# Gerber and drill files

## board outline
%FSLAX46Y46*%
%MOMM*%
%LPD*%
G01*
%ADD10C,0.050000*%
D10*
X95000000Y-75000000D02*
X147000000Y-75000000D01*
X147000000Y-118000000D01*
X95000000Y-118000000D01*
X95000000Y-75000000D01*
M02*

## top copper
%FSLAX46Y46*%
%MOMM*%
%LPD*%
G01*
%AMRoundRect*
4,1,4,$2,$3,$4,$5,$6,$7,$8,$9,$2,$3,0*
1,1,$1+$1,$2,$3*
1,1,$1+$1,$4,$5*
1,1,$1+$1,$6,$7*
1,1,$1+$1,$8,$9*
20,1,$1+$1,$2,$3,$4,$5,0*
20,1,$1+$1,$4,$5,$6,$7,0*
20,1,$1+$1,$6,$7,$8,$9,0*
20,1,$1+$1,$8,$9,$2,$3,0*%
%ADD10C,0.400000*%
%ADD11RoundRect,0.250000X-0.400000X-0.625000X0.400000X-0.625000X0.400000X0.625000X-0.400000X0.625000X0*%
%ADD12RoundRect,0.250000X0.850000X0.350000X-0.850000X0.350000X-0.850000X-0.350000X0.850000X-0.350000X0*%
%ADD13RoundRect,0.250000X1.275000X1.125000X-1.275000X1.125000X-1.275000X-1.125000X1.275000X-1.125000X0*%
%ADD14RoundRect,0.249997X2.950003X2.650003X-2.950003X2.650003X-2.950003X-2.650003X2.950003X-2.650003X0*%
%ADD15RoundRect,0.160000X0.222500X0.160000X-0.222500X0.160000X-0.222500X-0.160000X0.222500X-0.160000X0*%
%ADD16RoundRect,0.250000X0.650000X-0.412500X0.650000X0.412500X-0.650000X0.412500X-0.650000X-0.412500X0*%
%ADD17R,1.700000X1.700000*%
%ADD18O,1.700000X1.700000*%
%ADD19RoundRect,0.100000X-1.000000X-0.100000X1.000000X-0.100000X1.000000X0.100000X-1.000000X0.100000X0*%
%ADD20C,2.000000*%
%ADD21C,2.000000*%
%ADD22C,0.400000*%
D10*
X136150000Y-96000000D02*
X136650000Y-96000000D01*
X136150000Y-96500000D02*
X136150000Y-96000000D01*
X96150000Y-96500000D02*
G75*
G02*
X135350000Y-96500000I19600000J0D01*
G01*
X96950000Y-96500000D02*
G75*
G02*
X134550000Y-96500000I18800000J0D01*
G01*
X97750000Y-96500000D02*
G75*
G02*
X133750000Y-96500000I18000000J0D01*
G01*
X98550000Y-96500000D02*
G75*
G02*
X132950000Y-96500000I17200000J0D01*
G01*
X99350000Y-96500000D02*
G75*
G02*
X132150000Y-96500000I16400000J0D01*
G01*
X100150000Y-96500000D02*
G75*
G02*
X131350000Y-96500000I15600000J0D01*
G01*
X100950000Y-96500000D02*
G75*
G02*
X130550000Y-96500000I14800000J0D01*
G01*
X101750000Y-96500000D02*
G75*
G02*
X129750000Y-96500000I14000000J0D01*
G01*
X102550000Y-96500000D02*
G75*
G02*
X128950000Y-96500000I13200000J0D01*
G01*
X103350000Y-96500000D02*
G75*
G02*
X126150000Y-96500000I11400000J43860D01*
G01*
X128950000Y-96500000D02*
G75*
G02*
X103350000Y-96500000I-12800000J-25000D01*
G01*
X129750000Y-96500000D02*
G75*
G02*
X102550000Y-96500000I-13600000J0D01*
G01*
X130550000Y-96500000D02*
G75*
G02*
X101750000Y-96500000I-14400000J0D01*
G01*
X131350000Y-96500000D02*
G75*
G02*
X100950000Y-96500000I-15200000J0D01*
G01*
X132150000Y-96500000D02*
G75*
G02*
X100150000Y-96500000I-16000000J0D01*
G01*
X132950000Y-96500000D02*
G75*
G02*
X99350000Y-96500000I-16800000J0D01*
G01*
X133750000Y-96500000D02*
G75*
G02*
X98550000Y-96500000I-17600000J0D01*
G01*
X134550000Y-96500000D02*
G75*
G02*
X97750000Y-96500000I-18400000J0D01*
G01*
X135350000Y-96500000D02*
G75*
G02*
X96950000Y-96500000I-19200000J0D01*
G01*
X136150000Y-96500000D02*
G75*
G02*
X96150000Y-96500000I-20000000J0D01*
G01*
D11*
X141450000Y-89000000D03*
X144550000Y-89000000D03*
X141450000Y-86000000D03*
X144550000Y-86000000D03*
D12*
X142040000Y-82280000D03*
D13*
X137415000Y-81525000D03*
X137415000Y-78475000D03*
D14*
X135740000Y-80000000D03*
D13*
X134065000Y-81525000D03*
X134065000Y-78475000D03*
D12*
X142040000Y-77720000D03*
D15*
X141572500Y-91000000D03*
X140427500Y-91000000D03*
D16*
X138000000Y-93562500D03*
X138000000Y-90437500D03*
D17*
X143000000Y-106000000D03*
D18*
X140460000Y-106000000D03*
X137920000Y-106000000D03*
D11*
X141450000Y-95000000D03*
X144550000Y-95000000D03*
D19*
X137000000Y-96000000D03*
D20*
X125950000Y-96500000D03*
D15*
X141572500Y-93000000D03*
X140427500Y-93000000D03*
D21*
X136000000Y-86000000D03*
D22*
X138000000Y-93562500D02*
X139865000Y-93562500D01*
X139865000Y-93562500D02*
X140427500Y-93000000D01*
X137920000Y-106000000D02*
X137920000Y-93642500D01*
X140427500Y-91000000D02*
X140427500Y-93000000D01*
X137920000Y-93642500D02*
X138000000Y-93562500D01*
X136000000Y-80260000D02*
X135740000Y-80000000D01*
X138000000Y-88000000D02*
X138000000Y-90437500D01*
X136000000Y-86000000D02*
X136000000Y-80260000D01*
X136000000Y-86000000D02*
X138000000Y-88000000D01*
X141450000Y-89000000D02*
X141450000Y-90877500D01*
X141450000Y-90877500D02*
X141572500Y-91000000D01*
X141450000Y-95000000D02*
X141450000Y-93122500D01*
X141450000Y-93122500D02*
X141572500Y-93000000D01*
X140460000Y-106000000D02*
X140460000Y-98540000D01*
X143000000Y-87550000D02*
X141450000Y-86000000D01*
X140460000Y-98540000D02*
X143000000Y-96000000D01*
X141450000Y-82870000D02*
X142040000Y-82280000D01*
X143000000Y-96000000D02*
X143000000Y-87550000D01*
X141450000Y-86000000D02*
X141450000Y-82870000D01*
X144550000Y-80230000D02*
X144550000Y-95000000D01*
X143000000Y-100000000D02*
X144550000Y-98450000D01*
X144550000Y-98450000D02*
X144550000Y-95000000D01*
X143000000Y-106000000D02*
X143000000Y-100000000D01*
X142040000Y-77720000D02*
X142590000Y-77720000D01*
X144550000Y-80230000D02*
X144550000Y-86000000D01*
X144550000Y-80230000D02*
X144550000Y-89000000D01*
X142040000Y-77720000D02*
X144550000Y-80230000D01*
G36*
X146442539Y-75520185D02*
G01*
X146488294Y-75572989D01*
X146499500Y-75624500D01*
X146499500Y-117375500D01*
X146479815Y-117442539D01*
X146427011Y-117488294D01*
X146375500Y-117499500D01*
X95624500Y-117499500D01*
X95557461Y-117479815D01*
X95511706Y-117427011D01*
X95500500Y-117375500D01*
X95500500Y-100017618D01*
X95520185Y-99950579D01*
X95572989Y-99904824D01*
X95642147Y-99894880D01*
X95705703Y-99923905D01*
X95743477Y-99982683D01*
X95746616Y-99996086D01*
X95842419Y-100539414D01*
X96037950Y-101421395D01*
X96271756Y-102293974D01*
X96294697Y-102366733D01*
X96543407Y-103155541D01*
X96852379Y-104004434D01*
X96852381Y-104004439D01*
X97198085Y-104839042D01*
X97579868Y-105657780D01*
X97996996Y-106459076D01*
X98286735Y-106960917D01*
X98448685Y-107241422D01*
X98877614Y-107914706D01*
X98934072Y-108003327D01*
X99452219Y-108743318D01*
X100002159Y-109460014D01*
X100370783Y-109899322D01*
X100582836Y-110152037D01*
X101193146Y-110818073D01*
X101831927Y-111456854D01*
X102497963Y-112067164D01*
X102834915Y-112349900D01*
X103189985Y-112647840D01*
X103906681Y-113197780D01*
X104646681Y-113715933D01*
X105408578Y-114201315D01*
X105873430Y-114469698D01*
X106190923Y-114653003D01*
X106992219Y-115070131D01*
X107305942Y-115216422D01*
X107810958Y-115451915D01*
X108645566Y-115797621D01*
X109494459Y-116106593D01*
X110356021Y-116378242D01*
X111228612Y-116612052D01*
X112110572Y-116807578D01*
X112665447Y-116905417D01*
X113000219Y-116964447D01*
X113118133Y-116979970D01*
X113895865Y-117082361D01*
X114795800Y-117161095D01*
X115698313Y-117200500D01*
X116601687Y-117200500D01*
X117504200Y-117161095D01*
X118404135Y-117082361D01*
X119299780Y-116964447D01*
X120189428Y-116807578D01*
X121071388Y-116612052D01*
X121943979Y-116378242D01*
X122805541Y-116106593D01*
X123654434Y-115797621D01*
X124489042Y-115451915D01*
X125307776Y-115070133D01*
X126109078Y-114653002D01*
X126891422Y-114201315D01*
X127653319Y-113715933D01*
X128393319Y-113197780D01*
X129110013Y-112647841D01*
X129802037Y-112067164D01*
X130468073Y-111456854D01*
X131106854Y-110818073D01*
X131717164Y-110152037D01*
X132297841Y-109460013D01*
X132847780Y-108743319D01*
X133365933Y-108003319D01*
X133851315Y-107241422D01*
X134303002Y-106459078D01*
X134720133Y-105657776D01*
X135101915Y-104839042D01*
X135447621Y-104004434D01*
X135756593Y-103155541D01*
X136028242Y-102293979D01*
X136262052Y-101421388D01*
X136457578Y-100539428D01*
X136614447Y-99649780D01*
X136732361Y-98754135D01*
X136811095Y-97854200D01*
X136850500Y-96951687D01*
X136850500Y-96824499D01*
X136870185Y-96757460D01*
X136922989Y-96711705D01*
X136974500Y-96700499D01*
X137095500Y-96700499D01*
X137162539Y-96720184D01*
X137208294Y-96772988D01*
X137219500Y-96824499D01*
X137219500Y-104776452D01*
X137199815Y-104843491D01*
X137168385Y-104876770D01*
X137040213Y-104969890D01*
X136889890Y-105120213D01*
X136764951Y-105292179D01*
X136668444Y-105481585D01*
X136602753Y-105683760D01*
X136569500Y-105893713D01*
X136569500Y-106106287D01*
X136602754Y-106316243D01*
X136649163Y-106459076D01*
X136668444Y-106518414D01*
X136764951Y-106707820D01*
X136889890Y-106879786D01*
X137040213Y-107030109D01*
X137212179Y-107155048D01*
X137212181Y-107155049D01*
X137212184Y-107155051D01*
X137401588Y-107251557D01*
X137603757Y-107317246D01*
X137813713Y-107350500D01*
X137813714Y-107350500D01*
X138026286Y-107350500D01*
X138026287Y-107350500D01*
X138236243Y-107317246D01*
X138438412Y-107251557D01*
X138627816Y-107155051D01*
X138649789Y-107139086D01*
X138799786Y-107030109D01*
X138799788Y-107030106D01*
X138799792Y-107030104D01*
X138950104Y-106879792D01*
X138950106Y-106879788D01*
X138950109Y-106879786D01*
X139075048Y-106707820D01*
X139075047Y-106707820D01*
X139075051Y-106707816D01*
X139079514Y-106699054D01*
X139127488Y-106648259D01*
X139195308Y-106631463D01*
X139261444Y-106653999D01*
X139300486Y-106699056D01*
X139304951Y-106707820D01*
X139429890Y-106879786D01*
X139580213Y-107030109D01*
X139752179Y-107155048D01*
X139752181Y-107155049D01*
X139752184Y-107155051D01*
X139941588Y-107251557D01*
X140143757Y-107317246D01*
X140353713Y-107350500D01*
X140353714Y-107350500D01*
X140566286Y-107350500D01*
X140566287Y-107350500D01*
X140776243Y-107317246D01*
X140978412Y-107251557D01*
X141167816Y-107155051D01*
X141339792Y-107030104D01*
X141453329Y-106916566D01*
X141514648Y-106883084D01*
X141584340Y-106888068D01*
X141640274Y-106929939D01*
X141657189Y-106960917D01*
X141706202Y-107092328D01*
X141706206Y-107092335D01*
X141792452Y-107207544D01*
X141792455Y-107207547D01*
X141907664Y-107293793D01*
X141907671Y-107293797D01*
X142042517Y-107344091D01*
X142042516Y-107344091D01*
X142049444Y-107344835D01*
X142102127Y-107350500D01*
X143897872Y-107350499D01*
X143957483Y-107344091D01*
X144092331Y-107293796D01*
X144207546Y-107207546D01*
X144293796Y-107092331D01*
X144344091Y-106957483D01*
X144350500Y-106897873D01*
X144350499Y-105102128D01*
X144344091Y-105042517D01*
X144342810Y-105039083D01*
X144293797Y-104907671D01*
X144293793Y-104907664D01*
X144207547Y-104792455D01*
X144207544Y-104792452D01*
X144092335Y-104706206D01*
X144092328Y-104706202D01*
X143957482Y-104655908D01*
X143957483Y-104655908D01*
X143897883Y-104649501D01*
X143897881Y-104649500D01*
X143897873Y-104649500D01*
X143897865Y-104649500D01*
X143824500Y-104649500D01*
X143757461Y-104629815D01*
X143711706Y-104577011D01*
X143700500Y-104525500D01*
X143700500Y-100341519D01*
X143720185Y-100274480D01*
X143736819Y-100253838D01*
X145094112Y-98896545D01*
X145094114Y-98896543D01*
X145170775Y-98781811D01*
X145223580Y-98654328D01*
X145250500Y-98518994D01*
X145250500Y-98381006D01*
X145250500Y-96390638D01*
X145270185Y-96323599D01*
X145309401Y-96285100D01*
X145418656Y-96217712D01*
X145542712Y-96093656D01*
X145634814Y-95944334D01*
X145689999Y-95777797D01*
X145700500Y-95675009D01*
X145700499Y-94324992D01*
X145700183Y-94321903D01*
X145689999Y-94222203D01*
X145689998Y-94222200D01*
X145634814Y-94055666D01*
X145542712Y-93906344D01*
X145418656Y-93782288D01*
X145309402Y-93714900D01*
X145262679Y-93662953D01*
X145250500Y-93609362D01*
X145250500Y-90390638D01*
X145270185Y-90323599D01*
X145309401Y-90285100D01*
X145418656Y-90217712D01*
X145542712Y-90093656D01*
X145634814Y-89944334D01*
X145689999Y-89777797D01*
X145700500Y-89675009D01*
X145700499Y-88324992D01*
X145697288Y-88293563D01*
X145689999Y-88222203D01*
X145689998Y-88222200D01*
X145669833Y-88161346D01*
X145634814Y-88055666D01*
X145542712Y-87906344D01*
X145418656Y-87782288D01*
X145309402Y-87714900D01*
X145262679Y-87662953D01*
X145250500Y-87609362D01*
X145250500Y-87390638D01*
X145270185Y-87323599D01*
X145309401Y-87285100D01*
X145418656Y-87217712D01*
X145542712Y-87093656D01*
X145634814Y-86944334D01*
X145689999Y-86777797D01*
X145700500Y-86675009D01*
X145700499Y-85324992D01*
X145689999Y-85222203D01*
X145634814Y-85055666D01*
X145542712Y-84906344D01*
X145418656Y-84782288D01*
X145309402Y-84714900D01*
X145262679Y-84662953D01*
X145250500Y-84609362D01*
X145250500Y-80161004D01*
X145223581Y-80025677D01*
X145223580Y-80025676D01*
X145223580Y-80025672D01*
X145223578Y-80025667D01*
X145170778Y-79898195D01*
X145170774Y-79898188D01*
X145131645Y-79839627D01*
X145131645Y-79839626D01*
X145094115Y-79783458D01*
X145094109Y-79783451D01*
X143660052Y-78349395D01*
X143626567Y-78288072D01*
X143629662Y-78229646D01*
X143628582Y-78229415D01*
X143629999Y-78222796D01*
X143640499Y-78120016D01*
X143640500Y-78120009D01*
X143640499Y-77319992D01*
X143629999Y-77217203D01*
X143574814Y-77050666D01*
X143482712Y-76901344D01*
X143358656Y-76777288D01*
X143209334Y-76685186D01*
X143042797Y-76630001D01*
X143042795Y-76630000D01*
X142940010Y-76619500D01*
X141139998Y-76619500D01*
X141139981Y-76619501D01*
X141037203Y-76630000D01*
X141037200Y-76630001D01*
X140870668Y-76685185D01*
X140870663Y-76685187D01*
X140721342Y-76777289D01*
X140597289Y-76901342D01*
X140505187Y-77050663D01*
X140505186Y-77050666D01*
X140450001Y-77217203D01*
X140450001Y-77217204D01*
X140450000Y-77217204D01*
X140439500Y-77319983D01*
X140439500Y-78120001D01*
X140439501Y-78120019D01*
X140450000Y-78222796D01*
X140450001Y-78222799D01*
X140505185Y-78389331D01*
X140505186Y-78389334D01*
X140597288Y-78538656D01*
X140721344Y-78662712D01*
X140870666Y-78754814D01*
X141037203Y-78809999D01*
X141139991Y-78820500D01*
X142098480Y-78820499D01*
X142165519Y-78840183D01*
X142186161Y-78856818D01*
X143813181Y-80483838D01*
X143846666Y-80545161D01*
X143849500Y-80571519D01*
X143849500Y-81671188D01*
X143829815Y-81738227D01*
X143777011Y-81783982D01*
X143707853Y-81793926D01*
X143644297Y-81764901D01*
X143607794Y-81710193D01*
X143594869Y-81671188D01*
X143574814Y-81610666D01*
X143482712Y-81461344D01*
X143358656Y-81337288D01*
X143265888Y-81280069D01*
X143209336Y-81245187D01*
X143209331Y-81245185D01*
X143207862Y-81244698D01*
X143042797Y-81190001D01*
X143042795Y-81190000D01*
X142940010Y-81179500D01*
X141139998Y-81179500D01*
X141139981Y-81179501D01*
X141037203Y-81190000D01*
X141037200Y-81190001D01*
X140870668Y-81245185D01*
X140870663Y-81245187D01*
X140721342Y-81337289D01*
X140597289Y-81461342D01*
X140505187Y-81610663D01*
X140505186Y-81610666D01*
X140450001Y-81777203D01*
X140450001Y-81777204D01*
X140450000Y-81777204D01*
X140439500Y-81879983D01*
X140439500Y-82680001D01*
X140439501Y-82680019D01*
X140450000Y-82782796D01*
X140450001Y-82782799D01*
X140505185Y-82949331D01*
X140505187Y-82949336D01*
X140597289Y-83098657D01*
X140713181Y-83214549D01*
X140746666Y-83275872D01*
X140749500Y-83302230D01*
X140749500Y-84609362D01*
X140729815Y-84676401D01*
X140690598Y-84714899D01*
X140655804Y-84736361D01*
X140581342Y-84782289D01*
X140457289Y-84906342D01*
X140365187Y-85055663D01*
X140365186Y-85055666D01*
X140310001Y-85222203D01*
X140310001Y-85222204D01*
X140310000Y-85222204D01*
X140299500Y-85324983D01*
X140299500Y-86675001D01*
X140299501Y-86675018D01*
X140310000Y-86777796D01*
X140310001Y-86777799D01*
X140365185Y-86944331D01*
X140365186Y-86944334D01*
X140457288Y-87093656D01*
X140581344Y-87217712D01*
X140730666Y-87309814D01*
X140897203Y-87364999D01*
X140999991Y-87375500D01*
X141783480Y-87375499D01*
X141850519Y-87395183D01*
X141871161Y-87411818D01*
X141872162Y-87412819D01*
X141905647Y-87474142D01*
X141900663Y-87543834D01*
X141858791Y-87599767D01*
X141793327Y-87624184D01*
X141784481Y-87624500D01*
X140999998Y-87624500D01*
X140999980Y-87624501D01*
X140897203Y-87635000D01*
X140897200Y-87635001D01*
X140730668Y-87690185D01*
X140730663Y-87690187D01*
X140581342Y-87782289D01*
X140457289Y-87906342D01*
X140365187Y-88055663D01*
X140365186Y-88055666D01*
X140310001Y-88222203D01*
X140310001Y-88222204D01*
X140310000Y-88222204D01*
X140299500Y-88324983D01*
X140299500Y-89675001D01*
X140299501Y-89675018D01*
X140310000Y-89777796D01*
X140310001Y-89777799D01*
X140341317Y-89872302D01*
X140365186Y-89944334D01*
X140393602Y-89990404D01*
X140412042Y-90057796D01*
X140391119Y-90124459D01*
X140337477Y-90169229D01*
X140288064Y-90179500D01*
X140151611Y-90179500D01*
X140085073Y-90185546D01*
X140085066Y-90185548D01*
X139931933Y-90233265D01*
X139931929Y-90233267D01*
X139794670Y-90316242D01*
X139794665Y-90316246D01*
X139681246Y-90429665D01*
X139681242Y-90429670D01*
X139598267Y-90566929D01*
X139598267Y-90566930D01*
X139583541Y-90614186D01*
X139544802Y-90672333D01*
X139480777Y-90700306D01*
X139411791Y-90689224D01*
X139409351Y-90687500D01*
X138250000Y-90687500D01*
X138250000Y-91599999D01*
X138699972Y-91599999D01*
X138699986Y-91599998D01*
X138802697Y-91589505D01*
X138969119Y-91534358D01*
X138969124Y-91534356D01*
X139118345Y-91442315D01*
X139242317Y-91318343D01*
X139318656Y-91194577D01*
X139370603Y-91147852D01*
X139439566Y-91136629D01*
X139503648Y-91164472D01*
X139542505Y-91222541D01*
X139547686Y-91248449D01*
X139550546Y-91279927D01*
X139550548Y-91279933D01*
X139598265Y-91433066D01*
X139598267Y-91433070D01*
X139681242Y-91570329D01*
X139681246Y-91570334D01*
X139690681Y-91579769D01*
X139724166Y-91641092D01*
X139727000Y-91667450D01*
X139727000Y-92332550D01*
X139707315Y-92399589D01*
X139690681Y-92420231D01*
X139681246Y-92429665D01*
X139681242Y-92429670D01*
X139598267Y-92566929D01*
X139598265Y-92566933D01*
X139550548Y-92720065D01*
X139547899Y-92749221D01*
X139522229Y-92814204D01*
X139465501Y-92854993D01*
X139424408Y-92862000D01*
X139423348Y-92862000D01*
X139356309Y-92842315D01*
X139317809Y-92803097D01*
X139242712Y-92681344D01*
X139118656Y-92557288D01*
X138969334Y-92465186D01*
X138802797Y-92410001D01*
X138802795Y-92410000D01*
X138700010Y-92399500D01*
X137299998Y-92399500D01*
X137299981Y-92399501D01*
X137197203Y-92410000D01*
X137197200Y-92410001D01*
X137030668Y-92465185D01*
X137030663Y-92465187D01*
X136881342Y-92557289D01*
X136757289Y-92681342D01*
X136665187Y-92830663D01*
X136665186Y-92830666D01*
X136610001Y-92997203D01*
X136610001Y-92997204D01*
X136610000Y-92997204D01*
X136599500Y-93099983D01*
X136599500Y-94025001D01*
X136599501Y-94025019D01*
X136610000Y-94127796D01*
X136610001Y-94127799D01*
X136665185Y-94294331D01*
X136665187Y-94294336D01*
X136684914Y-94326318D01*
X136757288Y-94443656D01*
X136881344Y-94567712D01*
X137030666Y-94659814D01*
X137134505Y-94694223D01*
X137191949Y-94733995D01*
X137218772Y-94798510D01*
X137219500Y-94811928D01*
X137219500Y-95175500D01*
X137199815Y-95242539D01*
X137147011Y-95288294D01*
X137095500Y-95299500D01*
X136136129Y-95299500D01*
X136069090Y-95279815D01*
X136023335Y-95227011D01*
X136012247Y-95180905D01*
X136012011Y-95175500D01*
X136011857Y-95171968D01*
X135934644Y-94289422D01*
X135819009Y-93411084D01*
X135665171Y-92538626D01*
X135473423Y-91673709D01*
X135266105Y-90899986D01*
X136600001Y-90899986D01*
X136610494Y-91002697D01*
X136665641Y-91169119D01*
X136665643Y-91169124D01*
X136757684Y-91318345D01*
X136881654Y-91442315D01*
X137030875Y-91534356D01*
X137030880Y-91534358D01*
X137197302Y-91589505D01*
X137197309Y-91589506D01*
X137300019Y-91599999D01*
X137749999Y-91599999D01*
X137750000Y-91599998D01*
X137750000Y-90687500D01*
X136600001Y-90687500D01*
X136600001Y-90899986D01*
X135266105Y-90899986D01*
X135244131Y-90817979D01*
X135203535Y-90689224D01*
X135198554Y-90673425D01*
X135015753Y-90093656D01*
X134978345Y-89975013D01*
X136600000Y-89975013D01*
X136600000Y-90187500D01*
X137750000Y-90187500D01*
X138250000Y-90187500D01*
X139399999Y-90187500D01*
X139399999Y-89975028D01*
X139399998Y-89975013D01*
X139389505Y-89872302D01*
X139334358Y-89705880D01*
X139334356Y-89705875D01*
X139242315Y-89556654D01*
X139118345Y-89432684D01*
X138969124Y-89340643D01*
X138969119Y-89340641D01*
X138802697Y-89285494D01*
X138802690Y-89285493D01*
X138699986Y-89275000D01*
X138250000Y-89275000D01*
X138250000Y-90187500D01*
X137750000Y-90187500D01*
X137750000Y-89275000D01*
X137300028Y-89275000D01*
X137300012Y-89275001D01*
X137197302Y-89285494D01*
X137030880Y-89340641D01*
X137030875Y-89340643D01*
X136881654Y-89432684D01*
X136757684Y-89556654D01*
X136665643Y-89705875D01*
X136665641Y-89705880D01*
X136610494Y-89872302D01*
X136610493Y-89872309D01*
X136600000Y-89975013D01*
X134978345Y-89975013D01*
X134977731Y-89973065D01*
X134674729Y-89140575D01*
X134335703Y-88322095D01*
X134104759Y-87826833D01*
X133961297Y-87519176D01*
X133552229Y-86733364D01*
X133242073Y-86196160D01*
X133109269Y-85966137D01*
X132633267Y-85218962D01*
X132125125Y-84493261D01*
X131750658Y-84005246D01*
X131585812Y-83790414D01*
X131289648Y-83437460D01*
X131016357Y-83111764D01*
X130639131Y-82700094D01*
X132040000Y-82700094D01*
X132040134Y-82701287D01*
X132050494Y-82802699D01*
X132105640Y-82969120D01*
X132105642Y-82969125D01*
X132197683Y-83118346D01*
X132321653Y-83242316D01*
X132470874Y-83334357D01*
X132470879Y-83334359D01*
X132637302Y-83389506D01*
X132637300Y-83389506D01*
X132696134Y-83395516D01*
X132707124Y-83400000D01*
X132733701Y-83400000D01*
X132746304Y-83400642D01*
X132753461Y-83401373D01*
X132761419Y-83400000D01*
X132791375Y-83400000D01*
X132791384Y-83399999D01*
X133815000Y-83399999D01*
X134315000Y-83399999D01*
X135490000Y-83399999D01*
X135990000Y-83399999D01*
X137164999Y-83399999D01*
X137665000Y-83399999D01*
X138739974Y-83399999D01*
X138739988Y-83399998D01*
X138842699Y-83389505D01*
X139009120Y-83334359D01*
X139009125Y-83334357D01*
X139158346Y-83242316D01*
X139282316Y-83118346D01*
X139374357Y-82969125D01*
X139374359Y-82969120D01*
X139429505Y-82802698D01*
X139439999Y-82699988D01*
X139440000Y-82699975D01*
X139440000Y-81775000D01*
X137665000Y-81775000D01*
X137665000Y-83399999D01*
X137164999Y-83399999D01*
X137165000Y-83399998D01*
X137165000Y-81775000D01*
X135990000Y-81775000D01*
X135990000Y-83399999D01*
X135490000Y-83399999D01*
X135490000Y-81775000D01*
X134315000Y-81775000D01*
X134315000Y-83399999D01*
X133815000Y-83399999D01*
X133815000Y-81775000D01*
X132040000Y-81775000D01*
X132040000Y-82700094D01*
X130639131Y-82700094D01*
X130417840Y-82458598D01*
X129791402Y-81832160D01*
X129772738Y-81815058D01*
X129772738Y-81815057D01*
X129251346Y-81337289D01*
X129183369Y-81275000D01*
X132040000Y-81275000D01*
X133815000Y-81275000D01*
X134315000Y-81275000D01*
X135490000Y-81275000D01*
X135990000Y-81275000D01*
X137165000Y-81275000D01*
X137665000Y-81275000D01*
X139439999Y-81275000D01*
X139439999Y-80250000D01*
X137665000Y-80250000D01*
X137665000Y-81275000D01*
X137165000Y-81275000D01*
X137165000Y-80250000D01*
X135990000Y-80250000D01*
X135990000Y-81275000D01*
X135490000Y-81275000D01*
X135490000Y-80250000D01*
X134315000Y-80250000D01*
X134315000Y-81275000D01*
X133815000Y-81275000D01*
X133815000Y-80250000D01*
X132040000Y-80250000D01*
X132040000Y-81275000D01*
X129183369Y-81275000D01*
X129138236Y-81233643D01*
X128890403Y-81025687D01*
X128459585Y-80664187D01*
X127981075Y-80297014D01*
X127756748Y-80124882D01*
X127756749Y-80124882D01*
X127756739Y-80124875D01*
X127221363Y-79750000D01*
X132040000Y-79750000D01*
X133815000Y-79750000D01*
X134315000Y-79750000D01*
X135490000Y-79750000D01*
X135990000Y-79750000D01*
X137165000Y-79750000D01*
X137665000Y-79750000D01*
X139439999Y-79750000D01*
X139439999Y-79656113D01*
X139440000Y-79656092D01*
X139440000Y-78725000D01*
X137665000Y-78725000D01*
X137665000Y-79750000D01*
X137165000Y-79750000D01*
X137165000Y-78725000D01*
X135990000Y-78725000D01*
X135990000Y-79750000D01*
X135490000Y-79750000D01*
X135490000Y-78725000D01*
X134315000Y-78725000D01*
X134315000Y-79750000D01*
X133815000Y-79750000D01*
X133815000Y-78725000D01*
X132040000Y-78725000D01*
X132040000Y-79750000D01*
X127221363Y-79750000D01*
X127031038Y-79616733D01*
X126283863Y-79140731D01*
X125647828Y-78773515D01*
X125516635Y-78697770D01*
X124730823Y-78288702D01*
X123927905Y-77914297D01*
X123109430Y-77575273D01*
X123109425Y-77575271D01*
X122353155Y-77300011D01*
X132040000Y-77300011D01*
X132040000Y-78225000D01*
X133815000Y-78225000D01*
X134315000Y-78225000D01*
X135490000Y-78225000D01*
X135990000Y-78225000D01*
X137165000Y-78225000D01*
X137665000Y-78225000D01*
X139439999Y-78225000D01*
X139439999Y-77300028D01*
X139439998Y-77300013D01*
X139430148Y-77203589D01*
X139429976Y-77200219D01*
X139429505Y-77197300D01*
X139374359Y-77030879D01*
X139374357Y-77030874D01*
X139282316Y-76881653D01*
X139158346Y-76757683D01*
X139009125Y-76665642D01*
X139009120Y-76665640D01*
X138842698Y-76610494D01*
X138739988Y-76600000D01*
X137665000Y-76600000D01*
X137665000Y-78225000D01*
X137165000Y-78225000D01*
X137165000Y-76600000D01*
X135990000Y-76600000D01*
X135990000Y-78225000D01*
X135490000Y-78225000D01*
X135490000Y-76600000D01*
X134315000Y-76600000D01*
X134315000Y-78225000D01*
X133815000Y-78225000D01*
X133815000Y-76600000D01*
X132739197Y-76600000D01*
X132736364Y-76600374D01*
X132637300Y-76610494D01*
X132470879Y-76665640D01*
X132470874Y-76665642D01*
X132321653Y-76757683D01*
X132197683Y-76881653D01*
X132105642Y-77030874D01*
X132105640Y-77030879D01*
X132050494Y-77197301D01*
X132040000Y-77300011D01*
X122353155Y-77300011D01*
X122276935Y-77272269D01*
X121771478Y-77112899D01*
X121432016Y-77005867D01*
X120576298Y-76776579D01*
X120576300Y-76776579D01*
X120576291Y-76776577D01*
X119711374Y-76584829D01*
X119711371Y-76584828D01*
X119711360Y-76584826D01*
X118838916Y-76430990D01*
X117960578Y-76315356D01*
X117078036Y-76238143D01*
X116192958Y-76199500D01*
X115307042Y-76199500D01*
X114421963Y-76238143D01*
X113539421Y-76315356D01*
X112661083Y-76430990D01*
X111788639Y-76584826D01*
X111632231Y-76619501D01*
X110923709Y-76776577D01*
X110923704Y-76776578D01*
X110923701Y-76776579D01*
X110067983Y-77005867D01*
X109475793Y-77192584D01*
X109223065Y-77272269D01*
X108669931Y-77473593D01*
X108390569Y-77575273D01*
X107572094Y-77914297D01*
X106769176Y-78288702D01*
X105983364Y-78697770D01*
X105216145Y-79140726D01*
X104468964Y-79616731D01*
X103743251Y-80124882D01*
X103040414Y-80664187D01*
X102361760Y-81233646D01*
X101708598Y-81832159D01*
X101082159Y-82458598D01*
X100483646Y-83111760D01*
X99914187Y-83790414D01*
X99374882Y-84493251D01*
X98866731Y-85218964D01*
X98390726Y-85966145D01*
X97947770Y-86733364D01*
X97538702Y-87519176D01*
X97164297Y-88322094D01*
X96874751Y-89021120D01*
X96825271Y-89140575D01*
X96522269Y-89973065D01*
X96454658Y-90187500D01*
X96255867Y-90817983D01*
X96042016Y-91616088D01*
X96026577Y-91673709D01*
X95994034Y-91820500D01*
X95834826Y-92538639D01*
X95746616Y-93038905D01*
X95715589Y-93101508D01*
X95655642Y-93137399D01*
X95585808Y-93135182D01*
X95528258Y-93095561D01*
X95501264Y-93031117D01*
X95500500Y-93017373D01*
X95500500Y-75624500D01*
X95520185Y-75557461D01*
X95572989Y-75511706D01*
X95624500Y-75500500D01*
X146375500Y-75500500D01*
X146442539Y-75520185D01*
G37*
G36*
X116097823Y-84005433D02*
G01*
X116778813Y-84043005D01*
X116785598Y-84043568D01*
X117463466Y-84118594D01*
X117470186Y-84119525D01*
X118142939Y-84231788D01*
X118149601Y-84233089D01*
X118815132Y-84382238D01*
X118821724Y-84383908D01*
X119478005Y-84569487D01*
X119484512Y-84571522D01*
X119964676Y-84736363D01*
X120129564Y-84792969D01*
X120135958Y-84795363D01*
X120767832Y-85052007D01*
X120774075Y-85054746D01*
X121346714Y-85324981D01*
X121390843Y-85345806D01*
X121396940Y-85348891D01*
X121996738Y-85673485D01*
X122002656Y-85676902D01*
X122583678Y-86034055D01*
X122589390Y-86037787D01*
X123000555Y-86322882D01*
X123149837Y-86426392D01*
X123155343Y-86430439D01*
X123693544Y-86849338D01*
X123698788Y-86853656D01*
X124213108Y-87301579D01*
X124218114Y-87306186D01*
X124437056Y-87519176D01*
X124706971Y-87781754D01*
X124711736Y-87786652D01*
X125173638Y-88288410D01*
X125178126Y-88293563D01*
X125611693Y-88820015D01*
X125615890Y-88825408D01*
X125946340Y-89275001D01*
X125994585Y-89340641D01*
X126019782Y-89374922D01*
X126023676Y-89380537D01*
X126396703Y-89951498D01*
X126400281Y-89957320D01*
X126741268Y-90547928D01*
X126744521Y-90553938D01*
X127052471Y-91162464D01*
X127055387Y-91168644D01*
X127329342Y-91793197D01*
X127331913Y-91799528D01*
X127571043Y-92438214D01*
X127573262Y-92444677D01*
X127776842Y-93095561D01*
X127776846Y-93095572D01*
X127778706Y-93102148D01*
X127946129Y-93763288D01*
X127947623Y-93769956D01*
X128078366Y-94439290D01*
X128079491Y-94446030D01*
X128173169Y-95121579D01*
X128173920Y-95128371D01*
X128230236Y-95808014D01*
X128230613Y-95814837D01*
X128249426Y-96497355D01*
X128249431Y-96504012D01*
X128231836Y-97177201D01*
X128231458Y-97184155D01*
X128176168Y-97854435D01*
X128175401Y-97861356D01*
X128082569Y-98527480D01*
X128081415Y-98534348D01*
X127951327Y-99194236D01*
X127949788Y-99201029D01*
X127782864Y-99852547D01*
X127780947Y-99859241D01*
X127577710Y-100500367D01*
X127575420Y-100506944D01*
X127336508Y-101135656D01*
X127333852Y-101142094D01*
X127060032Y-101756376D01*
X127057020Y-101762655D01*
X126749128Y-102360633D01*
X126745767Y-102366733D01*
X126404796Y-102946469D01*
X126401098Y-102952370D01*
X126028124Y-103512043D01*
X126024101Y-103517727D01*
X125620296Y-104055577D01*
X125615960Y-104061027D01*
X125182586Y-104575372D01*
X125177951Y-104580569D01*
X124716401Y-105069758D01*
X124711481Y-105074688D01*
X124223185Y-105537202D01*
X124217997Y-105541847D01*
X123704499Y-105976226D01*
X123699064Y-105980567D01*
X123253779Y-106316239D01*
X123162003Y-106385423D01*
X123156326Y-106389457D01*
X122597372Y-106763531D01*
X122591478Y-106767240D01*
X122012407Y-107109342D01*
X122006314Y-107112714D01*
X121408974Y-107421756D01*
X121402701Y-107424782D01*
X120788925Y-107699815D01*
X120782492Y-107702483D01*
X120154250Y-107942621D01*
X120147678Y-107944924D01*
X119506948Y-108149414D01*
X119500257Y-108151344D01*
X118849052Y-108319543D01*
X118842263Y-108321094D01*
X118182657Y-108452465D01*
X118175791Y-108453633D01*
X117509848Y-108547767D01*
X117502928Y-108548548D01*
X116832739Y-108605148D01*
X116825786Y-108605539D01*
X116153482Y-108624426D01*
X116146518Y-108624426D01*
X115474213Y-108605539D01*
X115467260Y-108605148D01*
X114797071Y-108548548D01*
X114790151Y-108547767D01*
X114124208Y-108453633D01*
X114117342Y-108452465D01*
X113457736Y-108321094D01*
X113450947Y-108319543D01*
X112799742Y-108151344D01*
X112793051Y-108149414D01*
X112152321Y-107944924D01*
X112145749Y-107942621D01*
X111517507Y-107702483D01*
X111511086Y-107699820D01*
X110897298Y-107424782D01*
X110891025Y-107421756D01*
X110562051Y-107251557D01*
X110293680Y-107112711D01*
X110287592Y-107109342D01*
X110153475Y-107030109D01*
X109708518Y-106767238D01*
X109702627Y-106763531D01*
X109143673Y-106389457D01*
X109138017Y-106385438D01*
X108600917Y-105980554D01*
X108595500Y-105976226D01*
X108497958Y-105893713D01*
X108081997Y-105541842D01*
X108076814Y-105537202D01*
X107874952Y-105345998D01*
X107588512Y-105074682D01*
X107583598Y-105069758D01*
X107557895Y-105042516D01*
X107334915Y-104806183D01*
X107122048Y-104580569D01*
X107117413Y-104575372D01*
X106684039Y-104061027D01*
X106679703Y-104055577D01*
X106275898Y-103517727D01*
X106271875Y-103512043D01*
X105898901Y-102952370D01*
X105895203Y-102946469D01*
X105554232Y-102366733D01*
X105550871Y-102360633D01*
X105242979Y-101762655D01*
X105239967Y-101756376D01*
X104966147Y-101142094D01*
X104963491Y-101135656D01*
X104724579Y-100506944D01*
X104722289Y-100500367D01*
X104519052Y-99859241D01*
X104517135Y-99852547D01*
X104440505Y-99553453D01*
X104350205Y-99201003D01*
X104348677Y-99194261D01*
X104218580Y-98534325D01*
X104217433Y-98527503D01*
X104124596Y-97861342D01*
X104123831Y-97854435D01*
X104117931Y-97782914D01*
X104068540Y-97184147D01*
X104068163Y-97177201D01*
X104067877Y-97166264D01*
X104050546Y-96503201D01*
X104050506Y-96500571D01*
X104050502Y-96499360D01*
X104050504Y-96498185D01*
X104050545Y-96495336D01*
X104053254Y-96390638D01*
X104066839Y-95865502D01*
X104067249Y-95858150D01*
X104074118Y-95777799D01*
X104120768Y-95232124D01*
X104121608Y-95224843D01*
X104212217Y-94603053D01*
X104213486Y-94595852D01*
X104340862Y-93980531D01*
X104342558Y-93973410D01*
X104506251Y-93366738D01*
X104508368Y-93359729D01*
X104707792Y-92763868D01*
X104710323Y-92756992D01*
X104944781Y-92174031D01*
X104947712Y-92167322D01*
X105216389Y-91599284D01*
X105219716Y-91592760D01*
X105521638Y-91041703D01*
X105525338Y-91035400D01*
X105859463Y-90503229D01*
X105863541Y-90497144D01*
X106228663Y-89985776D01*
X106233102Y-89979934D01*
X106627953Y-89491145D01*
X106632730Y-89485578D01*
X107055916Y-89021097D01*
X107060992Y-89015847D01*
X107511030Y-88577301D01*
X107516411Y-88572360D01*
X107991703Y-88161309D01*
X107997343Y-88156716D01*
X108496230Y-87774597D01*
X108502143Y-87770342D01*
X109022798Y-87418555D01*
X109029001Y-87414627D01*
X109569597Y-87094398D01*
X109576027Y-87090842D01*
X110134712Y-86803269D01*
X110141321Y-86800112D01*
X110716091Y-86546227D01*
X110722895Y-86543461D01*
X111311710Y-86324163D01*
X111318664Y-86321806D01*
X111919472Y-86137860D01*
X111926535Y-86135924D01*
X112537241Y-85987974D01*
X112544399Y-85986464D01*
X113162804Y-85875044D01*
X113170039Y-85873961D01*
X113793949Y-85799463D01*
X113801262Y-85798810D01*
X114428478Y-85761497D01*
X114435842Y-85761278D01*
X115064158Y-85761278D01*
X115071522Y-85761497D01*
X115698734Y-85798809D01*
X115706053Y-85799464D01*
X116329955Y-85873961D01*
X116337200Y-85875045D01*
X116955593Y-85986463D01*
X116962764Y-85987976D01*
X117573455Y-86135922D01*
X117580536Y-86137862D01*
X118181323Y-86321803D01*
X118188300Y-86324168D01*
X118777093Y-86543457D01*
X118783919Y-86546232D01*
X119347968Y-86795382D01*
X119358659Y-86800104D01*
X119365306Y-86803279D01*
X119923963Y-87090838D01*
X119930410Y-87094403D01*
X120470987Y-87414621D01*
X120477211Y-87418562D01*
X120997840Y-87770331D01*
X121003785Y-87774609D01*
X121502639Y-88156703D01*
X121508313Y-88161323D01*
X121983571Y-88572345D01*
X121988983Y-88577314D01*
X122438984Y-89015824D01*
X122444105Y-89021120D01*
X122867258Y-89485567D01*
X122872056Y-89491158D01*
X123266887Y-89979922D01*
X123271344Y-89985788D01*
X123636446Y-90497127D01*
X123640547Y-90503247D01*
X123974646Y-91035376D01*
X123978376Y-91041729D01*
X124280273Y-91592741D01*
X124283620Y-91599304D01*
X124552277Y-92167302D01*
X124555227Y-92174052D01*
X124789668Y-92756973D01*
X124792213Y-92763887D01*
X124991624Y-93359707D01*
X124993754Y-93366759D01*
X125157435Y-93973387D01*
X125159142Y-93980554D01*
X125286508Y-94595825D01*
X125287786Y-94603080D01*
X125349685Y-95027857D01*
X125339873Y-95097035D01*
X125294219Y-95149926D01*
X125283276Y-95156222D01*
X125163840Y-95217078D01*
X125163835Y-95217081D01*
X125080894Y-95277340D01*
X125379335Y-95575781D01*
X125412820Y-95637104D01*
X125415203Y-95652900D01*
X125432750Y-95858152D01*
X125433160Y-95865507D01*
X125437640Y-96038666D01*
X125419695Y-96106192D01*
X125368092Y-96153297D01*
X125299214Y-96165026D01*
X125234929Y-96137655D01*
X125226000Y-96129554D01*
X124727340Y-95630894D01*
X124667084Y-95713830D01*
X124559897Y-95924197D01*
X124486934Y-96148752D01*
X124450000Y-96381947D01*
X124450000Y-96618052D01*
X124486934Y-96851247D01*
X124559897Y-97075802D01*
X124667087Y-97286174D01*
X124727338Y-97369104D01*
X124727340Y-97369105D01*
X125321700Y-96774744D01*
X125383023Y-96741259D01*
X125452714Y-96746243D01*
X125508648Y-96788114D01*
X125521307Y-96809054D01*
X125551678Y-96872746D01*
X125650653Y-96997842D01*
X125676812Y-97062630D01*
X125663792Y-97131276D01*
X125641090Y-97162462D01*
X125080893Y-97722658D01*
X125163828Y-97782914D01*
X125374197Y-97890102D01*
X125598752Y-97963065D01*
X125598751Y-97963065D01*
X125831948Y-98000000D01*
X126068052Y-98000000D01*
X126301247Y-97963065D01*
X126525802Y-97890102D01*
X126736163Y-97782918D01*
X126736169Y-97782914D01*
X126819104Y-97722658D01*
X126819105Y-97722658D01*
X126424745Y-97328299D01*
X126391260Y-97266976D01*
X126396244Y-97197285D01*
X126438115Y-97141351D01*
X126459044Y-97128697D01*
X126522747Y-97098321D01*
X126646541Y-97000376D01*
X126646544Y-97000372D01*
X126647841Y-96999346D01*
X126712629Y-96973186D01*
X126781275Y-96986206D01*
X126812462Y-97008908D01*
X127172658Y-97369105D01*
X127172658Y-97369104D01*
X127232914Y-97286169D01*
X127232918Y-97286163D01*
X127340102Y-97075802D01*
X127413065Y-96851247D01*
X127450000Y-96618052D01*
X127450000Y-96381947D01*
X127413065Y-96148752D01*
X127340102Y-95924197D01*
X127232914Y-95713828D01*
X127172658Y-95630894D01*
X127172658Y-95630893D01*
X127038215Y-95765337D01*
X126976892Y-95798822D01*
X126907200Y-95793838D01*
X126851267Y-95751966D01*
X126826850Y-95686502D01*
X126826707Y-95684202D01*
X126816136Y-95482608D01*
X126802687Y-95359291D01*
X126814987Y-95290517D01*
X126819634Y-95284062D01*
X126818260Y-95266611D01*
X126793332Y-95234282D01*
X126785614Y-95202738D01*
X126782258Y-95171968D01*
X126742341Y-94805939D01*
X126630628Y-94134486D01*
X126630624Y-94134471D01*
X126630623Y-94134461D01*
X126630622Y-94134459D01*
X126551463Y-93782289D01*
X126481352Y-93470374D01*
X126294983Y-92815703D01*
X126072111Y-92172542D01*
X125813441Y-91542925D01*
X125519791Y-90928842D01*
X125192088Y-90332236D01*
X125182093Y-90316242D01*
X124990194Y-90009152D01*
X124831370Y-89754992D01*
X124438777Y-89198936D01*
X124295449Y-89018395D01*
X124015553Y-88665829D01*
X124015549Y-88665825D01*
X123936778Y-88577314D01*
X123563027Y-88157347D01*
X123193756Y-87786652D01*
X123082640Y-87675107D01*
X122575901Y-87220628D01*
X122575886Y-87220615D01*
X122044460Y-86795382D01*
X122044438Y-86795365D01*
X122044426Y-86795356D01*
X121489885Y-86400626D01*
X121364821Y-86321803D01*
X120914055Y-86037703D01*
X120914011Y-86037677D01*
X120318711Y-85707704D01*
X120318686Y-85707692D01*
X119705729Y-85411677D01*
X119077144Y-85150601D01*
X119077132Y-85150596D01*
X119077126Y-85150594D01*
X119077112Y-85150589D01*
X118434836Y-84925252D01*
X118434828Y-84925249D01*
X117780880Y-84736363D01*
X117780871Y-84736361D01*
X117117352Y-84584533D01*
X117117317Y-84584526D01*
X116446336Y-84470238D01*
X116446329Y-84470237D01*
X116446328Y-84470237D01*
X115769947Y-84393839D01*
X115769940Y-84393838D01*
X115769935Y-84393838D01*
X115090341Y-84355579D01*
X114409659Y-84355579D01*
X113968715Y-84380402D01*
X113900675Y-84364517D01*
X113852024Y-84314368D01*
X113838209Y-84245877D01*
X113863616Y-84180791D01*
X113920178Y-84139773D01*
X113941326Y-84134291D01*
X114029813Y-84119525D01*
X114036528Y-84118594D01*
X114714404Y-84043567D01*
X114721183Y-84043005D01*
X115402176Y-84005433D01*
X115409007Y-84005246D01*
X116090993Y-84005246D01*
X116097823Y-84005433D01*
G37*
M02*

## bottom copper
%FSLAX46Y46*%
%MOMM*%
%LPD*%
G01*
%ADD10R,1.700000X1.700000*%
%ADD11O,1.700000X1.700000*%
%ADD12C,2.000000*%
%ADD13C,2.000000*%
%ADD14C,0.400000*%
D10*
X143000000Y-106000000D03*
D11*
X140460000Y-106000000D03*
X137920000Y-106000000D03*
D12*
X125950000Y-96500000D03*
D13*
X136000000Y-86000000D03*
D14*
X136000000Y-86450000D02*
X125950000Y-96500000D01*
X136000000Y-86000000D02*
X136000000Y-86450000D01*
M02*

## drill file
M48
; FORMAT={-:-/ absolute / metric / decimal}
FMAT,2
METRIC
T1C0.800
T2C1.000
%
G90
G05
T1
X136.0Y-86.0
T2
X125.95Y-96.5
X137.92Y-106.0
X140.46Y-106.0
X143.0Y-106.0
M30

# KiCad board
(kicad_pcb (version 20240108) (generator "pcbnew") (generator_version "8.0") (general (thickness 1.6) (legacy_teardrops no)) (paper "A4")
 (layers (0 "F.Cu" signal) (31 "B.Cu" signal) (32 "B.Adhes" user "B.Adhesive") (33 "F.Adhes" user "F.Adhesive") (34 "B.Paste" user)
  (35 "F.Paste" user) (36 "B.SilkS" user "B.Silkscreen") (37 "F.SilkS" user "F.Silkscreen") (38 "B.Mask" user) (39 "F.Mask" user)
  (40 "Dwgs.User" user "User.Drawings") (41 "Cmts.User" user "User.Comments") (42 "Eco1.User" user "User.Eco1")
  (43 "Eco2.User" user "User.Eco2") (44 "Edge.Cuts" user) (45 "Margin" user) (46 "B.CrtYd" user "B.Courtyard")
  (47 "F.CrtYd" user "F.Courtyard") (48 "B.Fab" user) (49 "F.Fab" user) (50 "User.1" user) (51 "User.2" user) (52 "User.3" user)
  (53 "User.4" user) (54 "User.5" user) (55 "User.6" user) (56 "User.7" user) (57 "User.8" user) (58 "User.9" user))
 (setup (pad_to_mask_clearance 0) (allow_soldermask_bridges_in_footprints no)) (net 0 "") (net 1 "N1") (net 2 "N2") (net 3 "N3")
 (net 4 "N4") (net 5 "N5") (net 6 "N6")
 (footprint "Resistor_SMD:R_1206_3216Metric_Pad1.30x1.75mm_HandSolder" (layer "F.Cu") (at 143 89)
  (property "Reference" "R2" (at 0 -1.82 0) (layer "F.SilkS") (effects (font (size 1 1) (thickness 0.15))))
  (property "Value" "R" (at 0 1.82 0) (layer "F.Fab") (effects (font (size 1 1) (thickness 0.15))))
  (pad "1" smd roundrect (at -1.55 0) (size 1.3 1.75) (layers "F.Cu" "F.Paste" "F.Mask") (roundrect_rratio 0.192308) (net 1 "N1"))
  (pad "2" smd roundrect (at 1.55 0) (size 1.3 1.75) (layers "F.Cu" "F.Paste" "F.Mask") (roundrect_rratio 0.192308) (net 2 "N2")))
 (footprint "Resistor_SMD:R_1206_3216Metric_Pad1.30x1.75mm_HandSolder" (layer "F.Cu") (at 143 86)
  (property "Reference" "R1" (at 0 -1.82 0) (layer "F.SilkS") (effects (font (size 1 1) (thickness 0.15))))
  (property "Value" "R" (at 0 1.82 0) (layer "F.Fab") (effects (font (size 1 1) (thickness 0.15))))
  (pad "1" smd roundrect (at -1.55 0) (size 1.3 1.75) (layers "F.Cu" "F.Paste" "F.Mask") (roundrect_rratio 0.192308) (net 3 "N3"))
  (pad "2" smd roundrect (at 1.55 0) (size 1.3 1.75) (layers "F.Cu" "F.Paste" "F.Mask") (roundrect_rratio 0.192308) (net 2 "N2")))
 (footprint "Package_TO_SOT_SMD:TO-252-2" (layer "F.Cu") (at 137 80 180)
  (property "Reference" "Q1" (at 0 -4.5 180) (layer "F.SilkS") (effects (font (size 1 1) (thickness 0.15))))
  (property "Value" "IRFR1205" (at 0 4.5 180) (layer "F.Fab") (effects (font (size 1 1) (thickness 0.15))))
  (pad "1" smd roundrect (at -5.04 -2.28 180) (size 2.2 1.2) (layers "F.Cu" "F.Paste" "F.Mask") (roundrect_rratio 0.208333) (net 3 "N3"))
  (pad "2" smd roundrect (at -0.415 -1.525 180) (size 3.05 2.75) (layers "F.Cu" "F.Paste") (roundrect_rratio 0.090909) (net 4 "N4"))
  (pad "2" smd roundrect (at -0.415 1.525 180) (size 3.05 2.75) (layers "F.Cu" "F.Paste") (roundrect_rratio 0.090909) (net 4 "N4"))
  (pad "2" smd roundrect (at 1.26 0 180) (size 6.4 5.8) (layers "F.Cu" "F.Mask") (roundrect_rratio 0.043103) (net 4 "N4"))
  (pad "2" smd roundrect (at 2.935 -1.525 180) (size 3.05 2.75) (layers "F.Cu" "F.Paste") (roundrect_rratio 0.090909) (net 4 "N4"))
  (pad "2" smd roundrect (at 2.935 1.525 180) (size 3.05 2.75) (layers "F.Cu" "F.Paste") (roundrect_rratio 0.090909) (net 4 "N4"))
  (pad "3" smd roundrect (at -5.04 2.28 180) (size 2.2 1.2) (layers "F.Cu" "F.Paste" "F.Mask") (roundrect_rratio 0.208333) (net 2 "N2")))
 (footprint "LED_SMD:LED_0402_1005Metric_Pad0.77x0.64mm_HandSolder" (layer "F.Cu") (at 141 91 180)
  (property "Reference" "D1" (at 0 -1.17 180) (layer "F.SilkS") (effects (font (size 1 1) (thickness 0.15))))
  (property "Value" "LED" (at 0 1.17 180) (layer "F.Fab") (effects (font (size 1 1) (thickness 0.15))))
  (pad "1" smd roundrect (at -0.5725 0 180) (size 0.765 0.64) (layers "F.Cu" "F.Paste" "F.Mask") (roundrect_rratio 0.25) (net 1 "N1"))
  (pad "2" smd roundrect (at 0.5725 0 180) (size 0.765 0.64) (layers "F.Cu" "F.Paste" "F.Mask") (roundrect_rratio 0.25) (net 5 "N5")))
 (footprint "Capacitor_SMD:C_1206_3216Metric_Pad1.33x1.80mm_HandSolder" (layer "F.Cu") (at 138 92 90)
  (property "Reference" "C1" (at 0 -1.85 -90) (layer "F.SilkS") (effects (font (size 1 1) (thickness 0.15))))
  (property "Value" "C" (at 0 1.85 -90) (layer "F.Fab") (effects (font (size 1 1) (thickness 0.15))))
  (pad "1" smd roundrect (at -1.5625 0 90) (size 1.325 1.8) (layers "F.Cu" "F.Paste" "F.Mask") (roundrect_rratio 0.188679) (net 5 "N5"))
  (pad "2" smd roundrect (at 1.5625 0 90) (size 1.325 1.8) (layers "F.Cu" "F.Paste" "F.Mask") (roundrect_rratio 0.188679) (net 4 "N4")))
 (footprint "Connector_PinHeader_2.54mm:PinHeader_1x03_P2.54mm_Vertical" (layer "F.Cu") (at 143 106 -90)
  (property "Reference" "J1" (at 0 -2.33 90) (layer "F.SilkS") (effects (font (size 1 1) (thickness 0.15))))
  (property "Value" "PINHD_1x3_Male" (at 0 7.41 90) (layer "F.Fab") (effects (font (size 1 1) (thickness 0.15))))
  (pad "1" thru_hole rect (at 0 0 270) (size 1.7 1.7) (drill 1) (layers "*.Cu" "*.Mask") (remove_unused_layers no) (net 2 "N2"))
  (pad "2" thru_hole oval (at 0 2.54 270) (size 1.7 1.7) (drill 1) (layers "*.Cu" "*.Mask") (remove_unused_layers no) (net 3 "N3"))
  (pad "3" thru_hole oval (at 0 5.08 270) (size 1.7 1.7) (drill 1) (layers "*.Cu" "*.Mask") (remove_unused_layers no) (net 5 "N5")))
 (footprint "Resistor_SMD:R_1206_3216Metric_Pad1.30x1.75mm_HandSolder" (layer "F.Cu") (at 143 95)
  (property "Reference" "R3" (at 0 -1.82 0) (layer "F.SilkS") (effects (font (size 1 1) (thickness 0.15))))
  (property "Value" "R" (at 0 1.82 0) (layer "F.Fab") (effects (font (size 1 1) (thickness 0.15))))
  (pad "1" smd roundrect (at -1.55 0) (size 1.3 1.75) (layers "F.Cu" "F.Paste" "F.Mask") (roundrect_rratio 0.192308) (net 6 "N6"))
  (pad "2" smd roundrect (at 1.55 0) (size 1.3 1.75) (layers "F.Cu" "F.Paste" "F.Mask") (roundrect_rratio 0.192308) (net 2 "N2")))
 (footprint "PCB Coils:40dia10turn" (layer "F.Cu") (at 115.75 96.5)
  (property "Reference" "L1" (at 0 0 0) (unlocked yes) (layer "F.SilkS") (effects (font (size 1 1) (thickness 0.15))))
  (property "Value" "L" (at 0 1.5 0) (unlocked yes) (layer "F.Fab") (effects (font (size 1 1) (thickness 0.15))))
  (fp_line (start 20.4 -0.5) (end 20.9 -0.5) (stroke (width 0.4) (type solid)) (layer "F.Cu"))
  (fp_line (start 20.4 0) (end 20.4 -0.5) (stroke (width 0.4) (type solid)) (layer "F.Cu"))
  (fp_arc (start -19.6 0) (mid 0 -19.6) (end 19.6 0) (stroke (width 0.4) (type solid)) (layer "F.Cu"))
  (fp_arc (start -18.8 0) (mid 0 -18.8) (end 18.8 0) (stroke (width 0.4) (type solid)) (layer "F.Cu"))
  (fp_arc (start -18 0) (mid 0 -18) (end 18 0) (stroke (width 0.4) (type solid)) (layer "F.Cu"))
  (fp_arc (start -17.2 0) (mid 0 -17.2) (end 17.2 0) (stroke (width 0.4) (type solid)) (layer "F.Cu"))
  (fp_arc (start -16.4 0) (mid 0 -16.4) (end 16.4 0) (stroke (width 0.4) (type solid)) (layer "F.Cu"))
  (fp_arc (start -15.6 0) (mid 0 -15.6) (end 15.6 0) (stroke (width 0.4) (type solid)) (layer "F.Cu"))
  (fp_arc (start -14.8 0) (mid 0 -14.8) (end 14.8 0) (stroke (width 0.4) (type solid)) (layer "F.Cu"))
  (fp_arc (start -14 0) (mid 0 -14) (end 14 0) (stroke (width 0.4) (type solid)) (layer "F.Cu"))
  (fp_arc (start -13.2 0) (mid 0 -13.2) (end 13.2 0) (stroke (width 0.4) (type solid)) (layer "F.Cu"))
  (fp_arc (start -12.4 0) (mid -1 -11.443944) (end 10.4 0) (stroke (width 0.4) (type solid)) (layer "F.Cu"))
  (fp_arc (start 13.2 0) (mid 0.4 12.825024) (end -12.4 0) (stroke (width 0.4) (type solid)) (layer "F.Cu"))
  (fp_arc (start 14 0) (mid 0.4 13.6) (end -13.2 0) (stroke (width 0.4) (type solid)) (layer "F.Cu"))
  (fp_arc (start 14.8 0) (mid 0.4 14.4) (end -14 0) (stroke (width 0.4) (type solid)) (layer "F.Cu"))
  (fp_arc (start 15.6 0) (mid 0.4 15.2) (end -14.8 0) (stroke (width 0.4) (type solid)) (layer "F.Cu"))
  (fp_arc (start 16.4 0) (mid 0.4 16) (end -15.6 0) (stroke (width 0.4) (type solid)) (layer "F.Cu"))
  (fp_arc (start 17.2 0) (mid 0.4 16.8) (end -16.4 0) (stroke (width 0.4) (type solid)) (layer "F.Cu"))
  (fp_arc (start 18 0) (mid 0.4 17.6) (end -17.2 0) (stroke (width 0.4) (type solid)) (layer "F.Cu"))
  (fp_arc (start 18.8 0) (mid 0.4 18.4) (end -18 0) (stroke (width 0.4) (type solid)) (layer "F.Cu"))
  (fp_arc (start 19.6 0) (mid 0.4 19.2) (end -18.8 0) (stroke (width 0.4) (type solid)) (layer "F.Cu"))
  (fp_arc (start 20.4 0) (mid 0.4 20) (end -19.6 0) (stroke (width 0.4) (type solid)) (layer "F.Cu"))
  (pad "1" smd roundrect (at 21.25 -0.5) (size 2.2 0.4) (layers "F.Cu") (roundrect_rratio 0.25) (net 5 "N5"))
  (pad "2" thru_hole circle (at 10.2 0) (size 2 2) (drill 1) (layers "*.Cu" "*.Mask") (remove_unused_layers no) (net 4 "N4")))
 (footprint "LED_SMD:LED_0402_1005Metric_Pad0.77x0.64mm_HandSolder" (layer "F.Cu") (at 141 93 180)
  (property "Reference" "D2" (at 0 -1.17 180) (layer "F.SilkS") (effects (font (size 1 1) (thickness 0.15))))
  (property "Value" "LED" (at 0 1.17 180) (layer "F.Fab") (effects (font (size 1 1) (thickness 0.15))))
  (pad "1" smd roundrect (at -0.5725 0 180) (size 0.765 0.64) (layers "F.Cu" "F.Paste" "F.Mask") (roundrect_rratio 0.25) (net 6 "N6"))
  (pad "2" smd roundrect (at 0.5725 0 180) (size 0.765 0.64) (layers "F.Cu" "F.Paste" "F.Mask") (roundrect_rratio 0.25) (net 5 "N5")))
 (gr_rect (start 95 75) (end 147 118) (stroke (width 0.05) (type default)) (fill none) (layer "Edge.Cuts"))
 (segment (start 138 93.5625) (end 139.865 93.5625) (width 0.4) (layer "F.Cu") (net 5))
 (segment (start 139.865 93.5625) (end 140.4275 93) (width 0.4) (layer "F.Cu") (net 5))
 (segment (start 137.92 106) (end 137.92 93.6425) (width 0.4) (layer "F.Cu") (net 5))
 (segment (start 140.4275 91) (end 140.4275 93) (width 0.4) (layer "F.Cu") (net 5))
 (segment (start 137.92 93.6425) (end 138 93.5625) (width 0.4) (layer "F.Cu") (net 5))
 (segment (start 136 80.26) (end 135.74 80) (width 0.4) (layer "F.Cu") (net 4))
 (segment (start 138 88) (end 138 90.4375) (width 0.4) (layer "F.Cu") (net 4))
 (segment (start 136 86) (end 136 80.26) (width 0.4) (layer "F.Cu") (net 4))
 (segment (start 136 86) (end 138 88) (width 0.4) (layer "F.Cu") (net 4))
 (via (at 136 86) (size 2) (drill 0.8) (layers "F.Cu" "B.Cu") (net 4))
 (segment (start 136 86.45) (end 125.95 96.5) (width 0.4) (layer "B.Cu") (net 4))
 (segment (start 136 86) (end 136 86.45) (width 0.4) (layer "B.Cu") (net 4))
 (segment (start 141.45 89) (end 141.45 90.8775) (width 0.4) (layer "F.Cu") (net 1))
 (segment (start 141.45 90.8775) (end 141.5725 91) (width 0.4) (layer "F.Cu") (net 1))
 (segment (start 141.45 95) (end 141.45 93.1225) (width 0.4) (layer "F.Cu") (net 6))
 (segment (start 141.45 93.1225) (end 141.5725 93) (width 0.4) (layer "F.Cu") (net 6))
 (segment (start 140.46 106) (end 140.46 98.54) (width 0.4) (layer "F.Cu") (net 3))
 (segment (start 143 87.55) (end 141.45 86) (width 0.4) (layer "F.Cu") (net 3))
 (segment (start 140.46 98.54) (end 143 96) (width 0.4) (layer "F.Cu") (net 3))
 (segment (start 141.45 82.87) (end 142.04 82.28) (width 0.4) (layer "F.Cu") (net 3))
 (segment (start 143 96) (end 143 87.55) (width 0.4) (layer "F.Cu") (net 3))
 (segment (start 141.45 86) (end 141.45 82.87) (width 0.4) (layer "F.Cu") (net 3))
 (segment (start 144.55 80.23) (end 144.55 95) (width 0.4) (layer "F.Cu") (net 2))
 (segment (start 143 100) (end 144.55 98.45) (width 0.4) (layer "F.Cu") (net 2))
 (segment (start 144.55 98.45) (end 144.55 95) (width 0.4) (layer "F.Cu") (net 2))
 (segment (start 143 106) (end 143 100) (width 0.4) (layer "F.Cu") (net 2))
 (segment (start 142.04 77.72) (end 142.59 77.72) (width 0.4) (layer "F.Cu") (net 2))
 (segment (start 144.55 80.23) (end 144.55 86) (width 0.4) (layer "F.Cu") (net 2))
 (segment (start 144.55 80.23) (end 144.55 89) (width 0.4) (layer "F.Cu") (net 2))
 (segment (start 142.04 77.72) (end 144.55 80.23) (width 0.4) (layer "F.Cu") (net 2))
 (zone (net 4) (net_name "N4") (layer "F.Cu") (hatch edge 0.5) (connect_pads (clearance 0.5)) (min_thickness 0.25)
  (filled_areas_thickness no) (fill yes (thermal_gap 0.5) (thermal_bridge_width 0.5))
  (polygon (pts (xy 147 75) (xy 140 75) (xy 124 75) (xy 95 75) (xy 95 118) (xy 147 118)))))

